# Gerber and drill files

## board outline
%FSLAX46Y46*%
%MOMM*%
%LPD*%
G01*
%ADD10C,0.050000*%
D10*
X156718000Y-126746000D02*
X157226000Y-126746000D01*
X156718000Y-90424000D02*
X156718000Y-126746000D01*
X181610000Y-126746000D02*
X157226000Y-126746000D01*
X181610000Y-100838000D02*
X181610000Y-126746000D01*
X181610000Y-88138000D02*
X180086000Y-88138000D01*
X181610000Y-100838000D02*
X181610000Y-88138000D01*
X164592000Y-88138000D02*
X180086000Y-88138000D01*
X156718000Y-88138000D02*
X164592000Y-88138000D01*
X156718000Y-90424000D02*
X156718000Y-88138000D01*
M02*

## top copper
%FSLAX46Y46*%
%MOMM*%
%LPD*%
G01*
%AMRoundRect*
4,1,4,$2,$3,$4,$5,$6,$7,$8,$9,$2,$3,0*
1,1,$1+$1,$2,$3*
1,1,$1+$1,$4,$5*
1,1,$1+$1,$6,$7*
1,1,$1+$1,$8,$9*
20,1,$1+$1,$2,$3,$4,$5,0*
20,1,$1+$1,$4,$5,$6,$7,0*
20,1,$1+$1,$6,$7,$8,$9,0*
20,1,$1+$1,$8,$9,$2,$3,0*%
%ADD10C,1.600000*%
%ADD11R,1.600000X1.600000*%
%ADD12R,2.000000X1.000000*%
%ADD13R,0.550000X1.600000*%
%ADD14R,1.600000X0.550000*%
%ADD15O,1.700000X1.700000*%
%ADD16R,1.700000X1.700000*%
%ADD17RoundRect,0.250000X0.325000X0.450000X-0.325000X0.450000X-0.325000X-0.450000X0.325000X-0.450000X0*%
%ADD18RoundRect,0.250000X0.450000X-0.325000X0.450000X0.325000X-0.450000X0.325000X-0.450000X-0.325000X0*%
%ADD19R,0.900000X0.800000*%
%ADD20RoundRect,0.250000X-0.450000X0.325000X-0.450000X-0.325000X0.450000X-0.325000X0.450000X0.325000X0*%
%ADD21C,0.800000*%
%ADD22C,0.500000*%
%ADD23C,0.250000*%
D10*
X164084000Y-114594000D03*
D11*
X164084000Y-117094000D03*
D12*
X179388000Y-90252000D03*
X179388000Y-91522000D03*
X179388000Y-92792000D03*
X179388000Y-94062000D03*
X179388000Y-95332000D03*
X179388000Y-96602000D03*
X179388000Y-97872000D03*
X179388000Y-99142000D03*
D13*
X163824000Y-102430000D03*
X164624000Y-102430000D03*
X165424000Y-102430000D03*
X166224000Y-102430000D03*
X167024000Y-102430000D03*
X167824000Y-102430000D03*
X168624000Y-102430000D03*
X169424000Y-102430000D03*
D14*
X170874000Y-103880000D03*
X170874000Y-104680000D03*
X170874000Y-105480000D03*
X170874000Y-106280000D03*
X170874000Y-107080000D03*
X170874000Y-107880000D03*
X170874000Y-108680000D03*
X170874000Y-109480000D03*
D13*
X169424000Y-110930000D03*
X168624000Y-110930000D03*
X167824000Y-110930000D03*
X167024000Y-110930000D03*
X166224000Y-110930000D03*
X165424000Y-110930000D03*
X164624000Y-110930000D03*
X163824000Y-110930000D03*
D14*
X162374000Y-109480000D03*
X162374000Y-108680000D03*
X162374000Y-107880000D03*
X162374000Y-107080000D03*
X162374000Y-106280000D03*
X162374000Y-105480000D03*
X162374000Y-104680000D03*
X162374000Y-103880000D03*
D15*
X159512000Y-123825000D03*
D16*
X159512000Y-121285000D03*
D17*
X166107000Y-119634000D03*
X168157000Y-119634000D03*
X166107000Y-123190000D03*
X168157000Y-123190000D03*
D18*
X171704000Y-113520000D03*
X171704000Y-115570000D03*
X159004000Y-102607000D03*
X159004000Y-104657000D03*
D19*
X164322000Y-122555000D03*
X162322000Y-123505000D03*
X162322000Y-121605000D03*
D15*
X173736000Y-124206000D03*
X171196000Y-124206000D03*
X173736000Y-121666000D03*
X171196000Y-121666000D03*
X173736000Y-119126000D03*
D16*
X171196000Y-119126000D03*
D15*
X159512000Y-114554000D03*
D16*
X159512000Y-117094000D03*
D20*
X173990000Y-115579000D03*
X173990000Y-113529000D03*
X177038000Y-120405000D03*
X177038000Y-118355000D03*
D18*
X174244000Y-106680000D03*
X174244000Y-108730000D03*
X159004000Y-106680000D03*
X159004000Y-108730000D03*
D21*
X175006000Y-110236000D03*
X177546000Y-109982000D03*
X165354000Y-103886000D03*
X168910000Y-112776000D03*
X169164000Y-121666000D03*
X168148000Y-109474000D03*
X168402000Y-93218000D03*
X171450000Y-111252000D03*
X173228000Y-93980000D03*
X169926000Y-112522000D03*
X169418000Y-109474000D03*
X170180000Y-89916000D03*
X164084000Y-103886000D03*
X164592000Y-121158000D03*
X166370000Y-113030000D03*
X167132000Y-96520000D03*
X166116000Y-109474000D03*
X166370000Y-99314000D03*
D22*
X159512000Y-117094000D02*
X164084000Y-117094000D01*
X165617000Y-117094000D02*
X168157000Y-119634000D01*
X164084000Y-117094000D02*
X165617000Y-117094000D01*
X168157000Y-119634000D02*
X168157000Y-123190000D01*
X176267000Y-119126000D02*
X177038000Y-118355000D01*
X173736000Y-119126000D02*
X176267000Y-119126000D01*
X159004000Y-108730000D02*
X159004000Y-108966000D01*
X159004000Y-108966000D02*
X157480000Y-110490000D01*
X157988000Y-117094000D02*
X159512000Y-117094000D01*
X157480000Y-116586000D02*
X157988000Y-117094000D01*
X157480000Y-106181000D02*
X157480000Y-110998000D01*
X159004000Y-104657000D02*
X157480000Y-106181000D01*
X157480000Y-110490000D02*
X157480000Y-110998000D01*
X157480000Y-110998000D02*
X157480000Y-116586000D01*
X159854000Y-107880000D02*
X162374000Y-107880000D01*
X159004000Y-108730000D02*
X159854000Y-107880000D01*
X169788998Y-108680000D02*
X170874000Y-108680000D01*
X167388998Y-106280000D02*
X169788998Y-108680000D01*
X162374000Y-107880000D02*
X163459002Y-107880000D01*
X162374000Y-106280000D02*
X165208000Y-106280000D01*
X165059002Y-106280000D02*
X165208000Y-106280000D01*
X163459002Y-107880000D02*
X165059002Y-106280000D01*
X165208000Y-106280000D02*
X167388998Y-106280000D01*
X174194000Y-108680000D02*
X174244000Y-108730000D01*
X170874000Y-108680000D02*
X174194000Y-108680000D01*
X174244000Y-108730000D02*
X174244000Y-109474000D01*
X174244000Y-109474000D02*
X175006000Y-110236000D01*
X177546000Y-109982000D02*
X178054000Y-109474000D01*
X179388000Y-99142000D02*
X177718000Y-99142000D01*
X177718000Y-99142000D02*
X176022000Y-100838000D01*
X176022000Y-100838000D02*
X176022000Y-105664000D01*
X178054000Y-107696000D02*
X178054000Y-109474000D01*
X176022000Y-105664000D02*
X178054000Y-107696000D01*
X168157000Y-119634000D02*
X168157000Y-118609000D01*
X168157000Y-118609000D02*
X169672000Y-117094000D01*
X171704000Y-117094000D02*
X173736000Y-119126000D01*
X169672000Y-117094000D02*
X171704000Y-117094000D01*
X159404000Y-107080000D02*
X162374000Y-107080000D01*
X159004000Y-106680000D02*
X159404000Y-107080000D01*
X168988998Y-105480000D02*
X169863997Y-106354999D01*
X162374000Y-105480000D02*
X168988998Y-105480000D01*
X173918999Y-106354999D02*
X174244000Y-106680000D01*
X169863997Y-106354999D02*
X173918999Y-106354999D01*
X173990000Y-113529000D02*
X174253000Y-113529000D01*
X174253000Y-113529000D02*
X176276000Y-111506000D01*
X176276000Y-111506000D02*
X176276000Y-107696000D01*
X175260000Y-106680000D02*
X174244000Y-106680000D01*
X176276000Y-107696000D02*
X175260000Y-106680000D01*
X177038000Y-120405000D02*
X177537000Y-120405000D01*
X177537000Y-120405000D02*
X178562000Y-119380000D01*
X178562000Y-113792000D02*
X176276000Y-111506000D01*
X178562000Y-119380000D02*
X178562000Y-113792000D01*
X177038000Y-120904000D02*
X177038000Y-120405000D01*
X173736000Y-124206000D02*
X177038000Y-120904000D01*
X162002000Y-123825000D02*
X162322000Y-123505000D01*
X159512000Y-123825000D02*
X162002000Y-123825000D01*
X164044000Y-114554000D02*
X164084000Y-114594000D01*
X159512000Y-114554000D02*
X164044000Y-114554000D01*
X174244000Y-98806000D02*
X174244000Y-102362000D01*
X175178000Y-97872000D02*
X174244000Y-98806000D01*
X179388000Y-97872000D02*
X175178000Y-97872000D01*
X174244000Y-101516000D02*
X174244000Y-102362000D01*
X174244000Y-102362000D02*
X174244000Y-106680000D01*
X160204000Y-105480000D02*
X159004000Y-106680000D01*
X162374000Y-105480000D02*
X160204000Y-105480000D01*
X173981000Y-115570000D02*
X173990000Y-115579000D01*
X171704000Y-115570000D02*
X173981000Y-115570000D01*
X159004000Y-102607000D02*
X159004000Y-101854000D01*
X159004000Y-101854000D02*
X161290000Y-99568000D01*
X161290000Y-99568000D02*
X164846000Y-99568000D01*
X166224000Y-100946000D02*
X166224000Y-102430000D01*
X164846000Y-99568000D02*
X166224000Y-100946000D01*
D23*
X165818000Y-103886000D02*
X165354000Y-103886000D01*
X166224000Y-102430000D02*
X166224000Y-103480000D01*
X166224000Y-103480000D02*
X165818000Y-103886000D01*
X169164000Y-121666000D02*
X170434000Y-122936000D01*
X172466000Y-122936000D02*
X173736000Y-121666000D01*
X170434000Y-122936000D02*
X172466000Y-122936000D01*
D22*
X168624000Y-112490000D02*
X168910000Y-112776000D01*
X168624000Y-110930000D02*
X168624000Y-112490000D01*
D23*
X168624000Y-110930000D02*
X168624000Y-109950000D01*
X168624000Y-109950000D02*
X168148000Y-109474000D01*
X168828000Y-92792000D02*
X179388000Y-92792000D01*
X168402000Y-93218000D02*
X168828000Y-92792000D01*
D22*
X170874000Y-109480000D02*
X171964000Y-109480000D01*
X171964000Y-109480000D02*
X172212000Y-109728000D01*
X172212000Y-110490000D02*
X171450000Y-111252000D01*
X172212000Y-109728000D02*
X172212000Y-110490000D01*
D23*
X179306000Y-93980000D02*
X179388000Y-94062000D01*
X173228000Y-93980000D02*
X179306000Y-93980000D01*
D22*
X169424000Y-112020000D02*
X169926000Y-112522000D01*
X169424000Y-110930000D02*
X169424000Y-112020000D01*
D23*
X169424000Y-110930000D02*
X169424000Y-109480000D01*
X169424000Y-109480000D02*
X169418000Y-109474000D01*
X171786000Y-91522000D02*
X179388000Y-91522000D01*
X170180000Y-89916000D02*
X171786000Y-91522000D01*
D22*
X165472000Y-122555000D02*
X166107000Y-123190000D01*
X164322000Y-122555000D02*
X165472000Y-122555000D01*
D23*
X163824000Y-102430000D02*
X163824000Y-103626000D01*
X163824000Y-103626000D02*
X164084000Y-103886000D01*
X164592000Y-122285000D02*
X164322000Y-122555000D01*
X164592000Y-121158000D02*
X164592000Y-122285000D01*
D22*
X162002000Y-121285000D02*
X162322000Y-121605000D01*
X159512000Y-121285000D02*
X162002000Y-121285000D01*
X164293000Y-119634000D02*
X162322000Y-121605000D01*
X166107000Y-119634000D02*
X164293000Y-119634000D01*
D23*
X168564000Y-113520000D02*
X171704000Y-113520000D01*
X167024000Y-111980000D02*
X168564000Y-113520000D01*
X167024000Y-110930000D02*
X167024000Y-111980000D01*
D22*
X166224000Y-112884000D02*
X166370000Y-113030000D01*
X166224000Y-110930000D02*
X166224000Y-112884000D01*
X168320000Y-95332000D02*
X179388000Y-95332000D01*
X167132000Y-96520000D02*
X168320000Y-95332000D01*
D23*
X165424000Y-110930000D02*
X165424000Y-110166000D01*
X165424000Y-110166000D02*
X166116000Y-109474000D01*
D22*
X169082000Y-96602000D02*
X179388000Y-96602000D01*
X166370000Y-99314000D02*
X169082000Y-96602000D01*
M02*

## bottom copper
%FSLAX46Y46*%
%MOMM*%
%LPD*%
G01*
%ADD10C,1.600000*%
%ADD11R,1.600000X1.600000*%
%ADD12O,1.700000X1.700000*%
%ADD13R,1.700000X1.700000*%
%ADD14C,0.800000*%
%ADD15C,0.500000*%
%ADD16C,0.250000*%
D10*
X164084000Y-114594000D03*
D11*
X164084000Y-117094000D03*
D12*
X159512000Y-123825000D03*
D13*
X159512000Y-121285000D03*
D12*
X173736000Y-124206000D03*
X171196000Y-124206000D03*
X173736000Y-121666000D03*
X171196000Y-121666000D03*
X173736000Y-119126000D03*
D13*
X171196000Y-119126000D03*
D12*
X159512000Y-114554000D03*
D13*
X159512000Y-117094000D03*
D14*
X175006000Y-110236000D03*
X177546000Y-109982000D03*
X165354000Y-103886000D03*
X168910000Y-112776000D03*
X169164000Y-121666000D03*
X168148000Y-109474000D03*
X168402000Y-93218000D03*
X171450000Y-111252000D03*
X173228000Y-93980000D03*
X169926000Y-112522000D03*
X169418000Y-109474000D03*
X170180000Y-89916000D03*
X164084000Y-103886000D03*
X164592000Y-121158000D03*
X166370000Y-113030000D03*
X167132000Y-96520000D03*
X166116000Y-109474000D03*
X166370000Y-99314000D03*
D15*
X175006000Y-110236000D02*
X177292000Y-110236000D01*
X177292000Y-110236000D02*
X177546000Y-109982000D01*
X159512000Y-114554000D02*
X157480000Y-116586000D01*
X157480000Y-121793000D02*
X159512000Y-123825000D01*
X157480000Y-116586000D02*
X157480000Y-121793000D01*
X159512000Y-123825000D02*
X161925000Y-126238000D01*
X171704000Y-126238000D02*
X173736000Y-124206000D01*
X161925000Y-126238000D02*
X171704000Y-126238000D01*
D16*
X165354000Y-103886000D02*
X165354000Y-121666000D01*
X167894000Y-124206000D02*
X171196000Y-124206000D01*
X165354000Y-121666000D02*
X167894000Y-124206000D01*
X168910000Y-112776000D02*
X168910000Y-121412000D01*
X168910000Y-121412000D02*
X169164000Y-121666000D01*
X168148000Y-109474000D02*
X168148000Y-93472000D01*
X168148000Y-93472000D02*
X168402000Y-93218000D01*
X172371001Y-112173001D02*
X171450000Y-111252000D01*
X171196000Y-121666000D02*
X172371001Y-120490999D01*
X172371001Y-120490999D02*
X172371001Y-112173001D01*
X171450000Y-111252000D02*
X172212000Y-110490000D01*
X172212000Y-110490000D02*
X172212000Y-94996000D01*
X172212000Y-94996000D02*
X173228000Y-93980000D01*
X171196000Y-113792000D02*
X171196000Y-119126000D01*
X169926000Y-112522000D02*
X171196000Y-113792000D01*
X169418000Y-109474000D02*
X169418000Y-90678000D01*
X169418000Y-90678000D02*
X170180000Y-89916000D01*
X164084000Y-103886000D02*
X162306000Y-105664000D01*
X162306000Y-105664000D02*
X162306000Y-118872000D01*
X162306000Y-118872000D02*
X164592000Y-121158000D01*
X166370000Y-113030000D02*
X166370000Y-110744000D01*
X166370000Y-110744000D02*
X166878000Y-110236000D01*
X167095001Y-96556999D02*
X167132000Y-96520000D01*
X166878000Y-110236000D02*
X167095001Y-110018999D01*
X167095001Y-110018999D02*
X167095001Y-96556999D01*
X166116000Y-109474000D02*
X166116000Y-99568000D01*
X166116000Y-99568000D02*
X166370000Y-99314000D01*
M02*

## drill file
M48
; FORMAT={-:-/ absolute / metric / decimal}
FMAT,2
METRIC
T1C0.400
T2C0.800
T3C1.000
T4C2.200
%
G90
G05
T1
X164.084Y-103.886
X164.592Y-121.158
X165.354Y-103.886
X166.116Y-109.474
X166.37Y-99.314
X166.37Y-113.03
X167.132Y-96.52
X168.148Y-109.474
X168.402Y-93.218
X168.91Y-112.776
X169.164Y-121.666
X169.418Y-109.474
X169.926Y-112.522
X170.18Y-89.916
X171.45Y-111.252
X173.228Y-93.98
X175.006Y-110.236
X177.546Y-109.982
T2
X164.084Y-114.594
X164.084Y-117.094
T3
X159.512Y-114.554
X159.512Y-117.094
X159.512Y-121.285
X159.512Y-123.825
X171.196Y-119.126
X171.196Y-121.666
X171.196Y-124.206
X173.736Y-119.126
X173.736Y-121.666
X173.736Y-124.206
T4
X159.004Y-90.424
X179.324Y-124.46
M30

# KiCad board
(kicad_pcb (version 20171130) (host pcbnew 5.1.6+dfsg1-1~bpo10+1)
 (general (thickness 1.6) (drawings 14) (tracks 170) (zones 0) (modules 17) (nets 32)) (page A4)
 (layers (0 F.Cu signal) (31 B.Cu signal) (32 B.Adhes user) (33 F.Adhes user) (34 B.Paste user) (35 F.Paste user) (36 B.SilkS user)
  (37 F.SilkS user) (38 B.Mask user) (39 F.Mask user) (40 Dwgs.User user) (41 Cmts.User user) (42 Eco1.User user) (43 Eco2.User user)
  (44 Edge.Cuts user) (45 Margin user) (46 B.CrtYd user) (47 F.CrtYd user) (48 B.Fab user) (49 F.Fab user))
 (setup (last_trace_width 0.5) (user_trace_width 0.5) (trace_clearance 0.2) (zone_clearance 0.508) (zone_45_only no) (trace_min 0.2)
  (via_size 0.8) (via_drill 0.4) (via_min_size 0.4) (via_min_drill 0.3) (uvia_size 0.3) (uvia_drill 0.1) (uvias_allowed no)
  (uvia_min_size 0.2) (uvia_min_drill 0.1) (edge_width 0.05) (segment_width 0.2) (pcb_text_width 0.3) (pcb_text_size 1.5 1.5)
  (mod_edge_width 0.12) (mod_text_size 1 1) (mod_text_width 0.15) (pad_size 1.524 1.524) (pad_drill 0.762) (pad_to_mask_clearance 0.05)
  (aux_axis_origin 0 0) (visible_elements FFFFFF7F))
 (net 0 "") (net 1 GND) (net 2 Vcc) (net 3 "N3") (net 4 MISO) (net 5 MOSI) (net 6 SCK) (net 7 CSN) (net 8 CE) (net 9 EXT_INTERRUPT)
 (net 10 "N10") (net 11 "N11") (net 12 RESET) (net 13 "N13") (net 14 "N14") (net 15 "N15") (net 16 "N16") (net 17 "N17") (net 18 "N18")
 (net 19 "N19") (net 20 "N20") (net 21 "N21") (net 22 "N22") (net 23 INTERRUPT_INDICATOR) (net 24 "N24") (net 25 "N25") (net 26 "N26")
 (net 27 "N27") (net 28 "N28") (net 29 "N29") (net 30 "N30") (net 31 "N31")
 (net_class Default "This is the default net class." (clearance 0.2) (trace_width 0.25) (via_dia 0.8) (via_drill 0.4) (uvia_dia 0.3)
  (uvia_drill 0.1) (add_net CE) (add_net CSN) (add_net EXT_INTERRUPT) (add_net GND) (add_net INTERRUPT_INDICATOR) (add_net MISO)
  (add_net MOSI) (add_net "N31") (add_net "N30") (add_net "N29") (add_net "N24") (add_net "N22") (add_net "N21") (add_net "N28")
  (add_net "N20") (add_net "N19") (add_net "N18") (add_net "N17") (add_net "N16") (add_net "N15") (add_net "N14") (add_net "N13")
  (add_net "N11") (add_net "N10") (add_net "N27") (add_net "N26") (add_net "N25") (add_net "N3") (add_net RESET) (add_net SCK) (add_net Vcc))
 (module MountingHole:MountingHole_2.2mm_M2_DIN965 (layer F.Cu) (at 179.324 124.46)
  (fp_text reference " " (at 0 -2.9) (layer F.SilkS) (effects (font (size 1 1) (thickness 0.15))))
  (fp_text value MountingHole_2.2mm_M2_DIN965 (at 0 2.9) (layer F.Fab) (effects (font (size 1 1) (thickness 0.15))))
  (pad 1 np_thru_hole circle (at 0 0) (size 2.2 2.2) (drill 2.2) (layers *.Cu *.Mask)))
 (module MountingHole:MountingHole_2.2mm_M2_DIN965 (layer F.Cu) (at 159.004 90.424)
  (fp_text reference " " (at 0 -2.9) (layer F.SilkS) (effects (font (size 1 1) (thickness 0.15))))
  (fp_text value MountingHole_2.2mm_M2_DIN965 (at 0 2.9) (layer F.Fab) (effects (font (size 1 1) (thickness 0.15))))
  (pad 1 np_thru_hole circle (at 0 0) (size 2.2 2.2) (drill 2.2) (layers *.Cu *.Mask)))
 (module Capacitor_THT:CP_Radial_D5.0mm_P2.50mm (layer F.Cu) (at 164.084 117.094 90)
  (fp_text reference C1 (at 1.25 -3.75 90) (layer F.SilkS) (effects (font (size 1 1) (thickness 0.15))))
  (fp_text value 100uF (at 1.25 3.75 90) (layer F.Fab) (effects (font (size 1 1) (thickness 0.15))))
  (pad 2 thru_hole circle (at 2.5 0 90) (size 1.6 1.6) (drill 0.8) (layers *.Cu *.Mask) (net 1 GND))
  (pad 1 thru_hole rect (at 0 0 90) (size 1.6 1.6) (drill 0.8) (layers *.Cu *.Mask) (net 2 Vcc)))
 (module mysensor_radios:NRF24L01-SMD (layer F.Cu) (at 170.688 94.742 90)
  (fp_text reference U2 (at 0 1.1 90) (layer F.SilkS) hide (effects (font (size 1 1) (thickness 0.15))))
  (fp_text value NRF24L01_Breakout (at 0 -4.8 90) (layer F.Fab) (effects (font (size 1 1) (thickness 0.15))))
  (pad 8 smd rect (at 4.49 8.7 90) (size 1 2) (layers F.Cu F.Paste F.Mask) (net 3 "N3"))
  (pad 7 smd rect (at 3.22 8.7 90) (size 1 2) (layers F.Cu F.Paste F.Mask) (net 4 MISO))
  (pad 6 smd rect (at 1.95 8.7 90) (size 1 2) (layers F.Cu F.Paste F.Mask) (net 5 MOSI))
  (pad 5 smd rect (at 0.68 8.7 90) (size 1 2) (layers F.Cu F.Paste F.Mask) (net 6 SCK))
  (pad 4 smd rect (at -0.59 8.7 90) (size 1 2) (layers F.Cu F.Paste F.Mask) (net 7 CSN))
  (pad 3 smd rect (at -1.86 8.7 90) (size 1 2) (layers F.Cu F.Paste F.Mask) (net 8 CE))
  (pad 1 smd rect (at -3.13 8.7 90) (size 1 2) (layers F.Cu F.Paste F.Mask) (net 1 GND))
  (pad 2 smd rect (at -4.4 8.7 90) (size 1 2) (layers F.Cu F.Paste F.Mask) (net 2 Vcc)))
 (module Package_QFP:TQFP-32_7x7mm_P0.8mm (layer F.Cu) (at 166.624 106.68)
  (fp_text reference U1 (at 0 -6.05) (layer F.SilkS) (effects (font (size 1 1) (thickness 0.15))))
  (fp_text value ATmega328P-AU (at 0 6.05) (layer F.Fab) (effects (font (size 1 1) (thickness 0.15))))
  (pad 32 smd rect (at -2.8 -4.25 90) (size 1.6 0.55) (layers F.Cu F.Paste F.Mask) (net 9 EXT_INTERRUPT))
  (pad 31 smd rect (at -2 -4.25 90) (size 1.6 0.55) (layers F.Cu F.Paste F.Mask) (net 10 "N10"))
  (pad 30 smd rect (at -1.2 -4.25 90) (size 1.6 0.55) (layers F.Cu F.Paste F.Mask) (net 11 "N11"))
  (pad 29 smd rect (at -0.4 -4.25 90) (size 1.6 0.55) (layers F.Cu F.Paste F.Mask) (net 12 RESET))
  (pad 28 smd rect (at 0.4 -4.25 90) (size 1.6 0.55) (layers F.Cu F.Paste F.Mask) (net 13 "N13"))
  (pad 27 smd rect (at 1.2 -4.25 90) (size 1.6 0.55) (layers F.Cu F.Paste F.Mask) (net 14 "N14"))
  (pad 26 smd rect (at 2 -4.25 90) (size 1.6 0.55) (layers F.Cu F.Paste F.Mask) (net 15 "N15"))
  (pad 25 smd rect (at 2.8 -4.25 90) (size 1.6 0.55) (layers F.Cu F.Paste F.Mask) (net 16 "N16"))
  (pad 24 smd rect (at 4.25 -2.8) (size 1.6 0.55) (layers F.Cu F.Paste F.Mask) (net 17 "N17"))
  (pad 23 smd rect (at 4.25 -2) (size 1.6 0.55) (layers F.Cu F.Paste F.Mask) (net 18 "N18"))
  (pad 22 smd rect (at 4.25 -1.2) (size 1.6 0.55) (layers F.Cu F.Paste F.Mask) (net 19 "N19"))
  (pad 21 smd rect (at 4.25 -0.4) (size 1.6 0.55) (layers F.Cu F.Paste F.Mask) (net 1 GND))
  (pad 20 smd rect (at 4.25 0.4) (size 1.6 0.55) (layers F.Cu F.Paste F.Mask) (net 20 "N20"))
  (pad 19 smd rect (at 4.25 1.2) (size 1.6 0.55) (layers F.Cu F.Paste F.Mask) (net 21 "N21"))
  (pad 18 smd rect (at 4.25 2) (size 1.6 0.55) (layers F.Cu F.Paste F.Mask) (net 2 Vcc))
  (pad 17 smd rect (at 4.25 2.8) (size 1.6 0.55) (layers F.Cu F.Paste F.Mask) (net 6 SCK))
  (pad 16 smd rect (at 2.8 4.25 90) (size 1.6 0.55) (layers F.Cu F.Paste F.Mask) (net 4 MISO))
  (pad 15 smd rect (at 2 4.25 90) (size 1.6 0.55) (layers F.Cu F.Paste F.Mask) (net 5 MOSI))
  (pad 14 smd rect (at 1.2 4.25 90) (size 1.6 0.55) (layers F.Cu F.Paste F.Mask) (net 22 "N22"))
  (pad 13 smd rect (at 0.4 4.25 90) (size 1.6 0.55) (layers F.Cu F.Paste F.Mask) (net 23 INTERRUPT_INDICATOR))
  (pad 12 smd rect (at -0.4 4.25 90) (size 1.6 0.55) (layers F.Cu F.Paste F.Mask) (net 7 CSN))
  (pad 11 smd rect (at -1.2 4.25 90) (size 1.6 0.55) (layers F.Cu F.Paste F.Mask) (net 8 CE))
  (pad 10 smd rect (at -2 4.25 90) (size 1.6 0.55) (layers F.Cu F.Paste F.Mask) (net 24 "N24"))
  (pad 9 smd rect (at -2.8 4.25 90) (size 1.6 0.55) (layers F.Cu F.Paste F.Mask) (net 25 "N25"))
  (pad 8 smd rect (at -4.25 2.8) (size 1.6 0.55) (layers F.Cu F.Paste F.Mask) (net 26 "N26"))
  (pad 7 smd rect (at -4.25 2) (size 1.6 0.55) (layers F.Cu F.Paste F.Mask) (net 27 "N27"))
  (pad 6 smd rect (at -4.25 1.2) (size 1.6 0.55) (layers F.Cu F.Paste F.Mask) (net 2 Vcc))
  (pad 5 smd rect (at -4.25 0.4) (size 1.6 0.55) (layers F.Cu F.Paste F.Mask) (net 1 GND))
  (pad 4 smd rect (at -4.25 -0.4) (size 1.6 0.55) (layers F.Cu F.Paste F.Mask) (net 2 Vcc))
  (pad 3 smd rect (at -4.25 -1.2) (size 1.6 0.55) (layers F.Cu F.Paste F.Mask) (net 1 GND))
  (pad 2 smd rect (at -4.25 -2) (size 1.6 0.55) (layers F.Cu F.Paste F.Mask) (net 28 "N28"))
  (pad 1 smd rect (at -4.25 -2.8) (size 1.6 0.55) (layers F.Cu F.Paste F.Mask) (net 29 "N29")))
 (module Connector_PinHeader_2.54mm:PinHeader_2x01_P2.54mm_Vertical (layer F.Cu) (at 159.512 121.285 270)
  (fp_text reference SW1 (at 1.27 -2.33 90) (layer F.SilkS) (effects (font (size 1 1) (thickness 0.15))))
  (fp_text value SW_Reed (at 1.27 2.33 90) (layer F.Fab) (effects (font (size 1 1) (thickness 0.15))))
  (pad 2 thru_hole oval (at 2.54 0 270) (size 1.7 1.7) (drill 1) (layers *.Cu *.Mask) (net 1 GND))
  (pad 1 thru_hole rect (at 0 0 270) (size 1.7 1.7) (drill 1) (layers *.Cu *.Mask) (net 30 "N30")))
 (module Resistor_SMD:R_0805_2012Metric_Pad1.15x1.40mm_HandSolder (layer F.Cu) (at 167.132 119.634 180)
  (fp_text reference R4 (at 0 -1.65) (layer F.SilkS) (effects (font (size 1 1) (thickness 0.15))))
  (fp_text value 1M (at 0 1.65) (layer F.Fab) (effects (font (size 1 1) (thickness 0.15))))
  (pad 2 smd roundrect (at 1.025 0 180) (size 1.15 1.4) (layers F.Cu F.Paste F.Mask) (roundrect_rratio 0.217391) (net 30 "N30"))
  (pad 1 smd roundrect (at -1.025 0 180) (size 1.15 1.4) (layers F.Cu F.Paste F.Mask) (roundrect_rratio 0.217391) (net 2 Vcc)))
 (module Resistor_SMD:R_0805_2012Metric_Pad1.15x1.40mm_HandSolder (layer F.Cu) (at 167.132 123.19 180)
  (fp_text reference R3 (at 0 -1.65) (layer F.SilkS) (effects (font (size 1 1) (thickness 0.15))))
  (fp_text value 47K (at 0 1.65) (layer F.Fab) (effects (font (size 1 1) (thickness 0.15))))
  (pad 2 smd roundrect (at 1.025 0 180) (size 1.15 1.4) (layers F.Cu F.Paste F.Mask) (roundrect_rratio 0.217391) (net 9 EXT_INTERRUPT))
  (pad 1 smd roundrect (at -1.025 0 180) (size 1.15 1.4) (layers F.Cu F.Paste F.Mask) (roundrect_rratio 0.217391) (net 2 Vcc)))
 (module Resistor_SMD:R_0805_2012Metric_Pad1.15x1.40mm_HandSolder (layer F.Cu) (at 171.704 114.545 90)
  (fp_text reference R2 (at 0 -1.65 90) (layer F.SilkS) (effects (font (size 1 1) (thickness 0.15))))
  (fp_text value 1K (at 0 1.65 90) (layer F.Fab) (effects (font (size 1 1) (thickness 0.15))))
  (pad 2 smd roundrect (at 1.025 0 90) (size 1.15 1.4) (layers F.Cu F.Paste F.Mask) (roundrect_rratio 0.217391) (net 23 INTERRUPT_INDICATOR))
  (pad 1 smd roundrect (at -1.025 0 90) (size 1.15 1.4) (layers F.Cu F.Paste F.Mask) (roundrect_rratio 0.217391) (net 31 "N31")))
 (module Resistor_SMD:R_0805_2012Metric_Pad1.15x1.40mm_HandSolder (layer F.Cu) (at 159.004 103.632 90)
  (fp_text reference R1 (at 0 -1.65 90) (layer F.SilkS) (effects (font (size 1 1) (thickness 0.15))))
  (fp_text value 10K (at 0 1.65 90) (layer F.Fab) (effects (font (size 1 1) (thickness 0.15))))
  (pad 2 smd roundrect (at 1.025 0 90) (size 1.15 1.4) (layers F.Cu F.Paste F.Mask) (roundrect_rratio 0.217391) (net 12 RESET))
  (pad 1 smd roundrect (at -1.025 0 90) (size 1.15 1.4) (layers F.Cu F.Paste F.Mask) (roundrect_rratio 0.217391) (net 2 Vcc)))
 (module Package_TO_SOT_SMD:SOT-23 (layer F.Cu) (at 163.322 122.555)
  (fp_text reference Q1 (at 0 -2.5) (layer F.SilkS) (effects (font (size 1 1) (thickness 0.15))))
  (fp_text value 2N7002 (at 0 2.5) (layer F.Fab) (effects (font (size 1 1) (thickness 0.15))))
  (pad 3 smd rect (at 1 0) (size 0.9 0.8) (layers F.Cu F.Paste F.Mask) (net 9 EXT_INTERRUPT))
  (pad 2 smd rect (at -1 0.95) (size 0.9 0.8) (layers F.Cu F.Paste F.Mask) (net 1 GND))
  (pad 1 smd rect (at -1 -0.95) (size 0.9 0.8) (layers F.Cu F.Paste F.Mask) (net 30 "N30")))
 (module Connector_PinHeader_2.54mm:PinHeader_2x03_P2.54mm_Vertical (layer F.Cu) (at 171.196 119.126)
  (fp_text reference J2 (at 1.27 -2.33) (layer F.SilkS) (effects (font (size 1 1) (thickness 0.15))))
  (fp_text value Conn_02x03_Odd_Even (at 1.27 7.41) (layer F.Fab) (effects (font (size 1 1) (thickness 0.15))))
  (pad 6 thru_hole oval (at 2.54 5.08) (size 1.7 1.7) (drill 1) (layers *.Cu *.Mask) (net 1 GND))
  (pad 5 thru_hole oval (at 0 5.08) (size 1.7 1.7) (drill 1) (layers *.Cu *.Mask) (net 12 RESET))
  (pad 4 thru_hole oval (at 2.54 2.54) (size 1.7 1.7) (drill 1) (layers *.Cu *.Mask) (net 5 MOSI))
  (pad 3 thru_hole oval (at 0 2.54) (size 1.7 1.7) (drill 1) (layers *.Cu *.Mask) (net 6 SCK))
  (pad 2 thru_hole oval (at 2.54 0) (size 1.7 1.7) (drill 1) (layers *.Cu *.Mask) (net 2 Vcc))
  (pad 1 thru_hole rect (at 0 0) (size 1.7 1.7) (drill 1) (layers *.Cu *.Mask) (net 4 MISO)))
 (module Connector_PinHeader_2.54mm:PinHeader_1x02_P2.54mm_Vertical (layer F.Cu) (at 159.512 117.094 180)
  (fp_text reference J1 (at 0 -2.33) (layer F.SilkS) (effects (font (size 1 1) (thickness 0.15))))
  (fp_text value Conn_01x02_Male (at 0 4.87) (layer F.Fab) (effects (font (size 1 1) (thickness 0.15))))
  (pad 2 thru_hole oval (at 0 2.54 180) (size 1.7 1.7) (drill 1) (layers *.Cu *.Mask) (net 1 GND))
  (pad 1 thru_hole rect (at 0 0 180) (size 1.7 1.7) (drill 1) (layers *.Cu *.Mask) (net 2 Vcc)))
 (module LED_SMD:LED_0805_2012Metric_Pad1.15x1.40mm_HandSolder (layer F.Cu) (at 173.99 114.554 270)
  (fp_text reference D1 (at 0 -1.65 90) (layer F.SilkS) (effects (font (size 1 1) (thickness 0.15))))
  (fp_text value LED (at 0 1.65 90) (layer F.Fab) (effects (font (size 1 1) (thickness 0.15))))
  (pad 2 smd roundrect (at 1.025 0 270) (size 1.15 1.4) (layers F.Cu F.Paste F.Mask) (roundrect_rratio 0.217391) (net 31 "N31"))
  (pad 1 smd roundrect (at -1.025 0 270) (size 1.15 1.4) (layers F.Cu F.Paste F.Mask) (roundrect_rratio 0.217391) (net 1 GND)))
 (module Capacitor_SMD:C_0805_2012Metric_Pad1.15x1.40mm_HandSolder (layer F.Cu) (at 177.038 119.38 270)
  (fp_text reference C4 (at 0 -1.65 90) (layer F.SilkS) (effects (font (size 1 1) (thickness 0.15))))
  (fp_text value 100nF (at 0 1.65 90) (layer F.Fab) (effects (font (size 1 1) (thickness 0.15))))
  (pad 2 smd roundrect (at 1.025 0 270) (size 1.15 1.4) (layers F.Cu F.Paste F.Mask) (roundrect_rratio 0.217391) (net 1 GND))
  (pad 1 smd roundrect (at -1.025 0 270) (size 1.15 1.4) (layers F.Cu F.Paste F.Mask) (roundrect_rratio 0.217391) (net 2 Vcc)))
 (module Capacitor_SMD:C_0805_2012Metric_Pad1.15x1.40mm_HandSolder (layer F.Cu) (at 174.244 107.705 90)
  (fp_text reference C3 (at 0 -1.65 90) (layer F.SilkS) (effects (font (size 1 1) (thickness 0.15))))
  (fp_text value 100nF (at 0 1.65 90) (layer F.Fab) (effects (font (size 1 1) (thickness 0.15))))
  (pad 2 smd roundrect (at 1.025 0 90) (size 1.15 1.4) (layers F.Cu F.Paste F.Mask) (roundrect_rratio 0.217391) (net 1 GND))
  (pad 1 smd roundrect (at -1.025 0 90) (size 1.15 1.4) (layers F.Cu F.Paste F.Mask) (roundrect_rratio 0.217391) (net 2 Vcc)))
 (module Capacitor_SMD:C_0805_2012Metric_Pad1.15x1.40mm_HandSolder (layer F.Cu) (at 159.004 107.705 90)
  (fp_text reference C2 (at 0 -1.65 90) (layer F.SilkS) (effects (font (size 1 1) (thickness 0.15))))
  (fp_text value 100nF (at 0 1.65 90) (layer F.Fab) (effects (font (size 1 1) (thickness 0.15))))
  (pad 2 smd roundrect (at 1.025 0 90) (size 1.15 1.4) (layers F.Cu F.Paste F.Mask) (roundrect_rratio 0.217391) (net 1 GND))
  (pad 1 smd roundrect (at -1.025 0 90) (size 1.15 1.4) (layers F.Cu F.Paste F.Mask) (roundrect_rratio 0.217391) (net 2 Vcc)))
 (gr_line (start 156.718 126.746) (end 157.226 126.746) (layer Edge.Cuts) (width 0.05))
 (gr_line (start 156.718 90.424) (end 156.718 126.746) (layer Edge.Cuts) (width 0.05))
 (gr_line (start 181.61 126.746) (end 157.226 126.746) (layer Edge.Cuts) (width 0.05))
 (gr_line (start 181.61 100.838) (end 181.61 126.746) (layer Edge.Cuts) (width 0.05))
 (gr_line (start 181.61 88.138) (end 180.086 88.138) (layer Edge.Cuts) (width 0.05))
 (gr_line (start 181.61 100.838) (end 181.61 88.138) (layer Edge.Cuts) (width 0.05))
 (gr_line (start 164.592 88.138) (end 180.086 88.138) (layer Edge.Cuts) (width 0.05))
 (gr_line (start 156.718 88.138) (end 164.592 88.138) (layer Edge.Cuts) (width 0.05))
 (gr_line (start 156.718 90.424) (end 156.718 88.138) (layer Edge.Cuts) (width 0.05))
 (segment (start 159.512 117.094) (end 164.084 117.094) (width 0.5) (layer F.Cu) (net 2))
 (segment (start 165.617 117.094) (end 168.157 119.634) (width 0.5) (layer F.Cu) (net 2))
 (segment (start 164.084 117.094) (end 165.617 117.094) (width 0.5) (layer F.Cu) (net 2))
 (segment (start 168.157 119.634) (end 168.157 123.19) (width 0.5) (layer F.Cu) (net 2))
 (segment (start 176.267 119.126) (end 177.038 118.355) (width 0.5) (layer F.Cu) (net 2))
 (segment (start 173.736 119.126) (end 176.267 119.126) (width 0.5) (layer F.Cu) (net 2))
 (segment (start 159.004 108.73) (end 159.004 108.966) (width 0.5) (layer F.Cu) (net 2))
 (segment (start 159.004 108.966) (end 157.48 110.49) (width 0.5) (layer F.Cu) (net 2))
 (segment (start 157.988 117.094) (end 159.512 117.094) (width 0.5) (layer F.Cu) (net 2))
 (segment (start 157.48 116.586) (end 157.988 117.094) (width 0.5) (layer F.Cu) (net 2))
 (segment (start 157.48 106.181) (end 157.48 110.998) (width 0.5) (layer F.Cu) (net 2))
 (segment (start 159.004 104.657) (end 157.48 106.181) (width 0.5) (layer F.Cu) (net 2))
 (segment (start 157.48 110.49) (end 157.48 110.998) (width 0.5) (layer F.Cu) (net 2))
 (segment (start 157.48 110.998) (end 157.48 116.586) (width 0.5) (layer F.Cu) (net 2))
 (segment (start 159.854 107.88) (end 162.374 107.88) (width 0.5) (layer F.Cu) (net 2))
 (segment (start 159.004 108.73) (end 159.854 107.88) (width 0.5) (layer F.Cu) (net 2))
 (segment (start 169.788998 108.68) (end 170.874 108.68) (width 0.5) (layer F.Cu) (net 2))
 (segment (start 167.388998 106.28) (end 169.788998 108.68) (width 0.5) (layer F.Cu) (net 2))
 (segment (start 162.374 107.88) (end 163.459002 107.88) (width 0.5) (layer F.Cu) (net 2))
 (segment (start 162.374 106.28) (end 165.208 106.28) (width 0.5) (layer F.Cu) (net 2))
 (segment (start 165.059002 106.28) (end 165.208 106.28) (width 0.5) (layer F.Cu) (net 2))
 (segment (start 163.459002 107.88) (end 165.059002 106.28) (width 0.5) (layer F.Cu) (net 2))
 (segment (start 165.208 106.28) (end 167.388998 106.28) (width 0.5) (layer F.Cu) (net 2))
 (segment (start 174.194 108.68) (end 174.244 108.73) (width 0.5) (layer F.Cu) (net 2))
 (segment (start 170.874 108.68) (end 174.194 108.68) (width 0.5) (layer F.Cu) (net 2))
 (segment (start 174.244 108.73) (end 174.244 109.474) (width 0.5) (layer F.Cu) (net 2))
 (via (at 175.006 110.236) (size 0.8) (drill 0.4) (layers F.Cu B.Cu) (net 2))
 (segment (start 174.244 109.474) (end 175.006 110.236) (width 0.5) (layer F.Cu) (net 2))
 (via (at 177.546 109.982) (size 0.8) (drill 0.4) (layers F.Cu B.Cu) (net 2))
 (segment (start 175.006 110.236) (end 177.292 110.236) (width 0.5) (layer B.Cu) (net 2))
 (segment (start 177.292 110.236) (end 177.546 109.982) (width 0.5) (layer B.Cu) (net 2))
 (segment (start 177.546 109.982) (end 178.054 109.474) (width 0.5) (layer F.Cu) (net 2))
 (segment (start 179.388 99.142) (end 177.718 99.142) (width 0.5) (layer F.Cu) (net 2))
 (segment (start 177.718 99.142) (end 176.022 100.838) (width 0.5) (layer F.Cu) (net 2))
 (segment (start 176.022 100.838) (end 176.022 105.664) (width 0.5) (layer F.Cu) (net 2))
 (segment (start 178.054 107.696) (end 178.054 109.474) (width 0.5) (layer F.Cu) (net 2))
 (segment (start 176.022 105.664) (end 178.054 107.696) (width 0.5) (layer F.Cu) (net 2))
 (segment (start 168.157 119.634) (end 168.157 118.609) (width 0.5) (layer F.Cu) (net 2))
 (segment (start 168.157 118.609) (end 169.672 117.094) (width 0.5) (layer F.Cu) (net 2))
 (segment (start 171.704 117.094) (end 173.736 119.126) (width 0.5) (layer F.Cu) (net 2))
 (segment (start 169.672 117.094) (end 171.704 117.094) (width 0.5) (layer F.Cu) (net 2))
 (segment (start 159.404 107.08) (end 162.374 107.08) (width 0.5) (layer F.Cu) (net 1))
 (segment (start 159.004 106.68) (end 159.404 107.08) (width 0.5) (layer F.Cu) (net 1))
 (segment (start 168.988998 105.48) (end 169.863997 106.354999) (width 0.5) (layer F.Cu) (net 1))
 (segment (start 162.374 105.48) (end 168.988998 105.48) (width 0.5) (layer F.Cu) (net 1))
 (segment (start 173.918999 106.354999) (end 174.244 106.68) (width 0.5) (layer F.Cu) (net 1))
 (segment (start 169.863997 106.354999) (end 173.918999 106.354999) (width 0.5) (layer F.Cu) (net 1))
 (segment (start 173.99 113.529) (end 174.253 113.529) (width 0.5) (layer F.Cu) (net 1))
 (segment (start 174.253 113.529) (end 176.276 111.506) (width 0.5) (layer F.Cu) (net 1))
 (segment (start 176.276 111.506) (end 176.276 107.696) (width 0.5) (layer F.Cu) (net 1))
 (segment (start 175.26 106.68) (end 174.244 106.68) (width 0.5) (layer F.Cu) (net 1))
 (segment (start 176.276 107.696) (end 175.26 106.68) (width 0.5) (layer F.Cu) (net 1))
 (segment (start 177.038 120.405) (end 177.537 120.405) (width 0.5) (layer F.Cu) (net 1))
 (segment (start 177.537 120.405) (end 178.562 119.38) (width 0.5) (layer F.Cu) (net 1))
 (segment (start 178.562 113.792) (end 176.276 111.506) (width 0.5) (layer F.Cu) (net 1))
 (segment (start 178.562 119.38) (end 178.562 113.792) (width 0.5) (layer F.Cu) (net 1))
 (segment (start 177.038 120.904) (end 177.038 120.405) (width 0.5) (layer F.Cu) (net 1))
 (segment (start 173.736 124.206) (end 177.038 120.904) (width 0.5) (layer F.Cu) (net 1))
 (segment (start 162.002 123.825) (end 162.322 123.505) (width 0.5) (layer F.Cu) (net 1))
 (segment (start 159.512 123.825) (end 162.002 123.825) (width 0.5) (layer F.Cu) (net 1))
 (segment (start 164.044 114.554) (end 164.084 114.594) (width 0.5) (layer F.Cu) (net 1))
 (segment (start 159.512 114.554) (end 164.044 114.554) (width 0.5) (layer F.Cu) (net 1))
 (segment (start 159.512 114.554) (end 157.48 116.586) (width 0.5) (layer B.Cu) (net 1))
 (segment (start 157.48 121.793) (end 159.512 123.825) (width 0.5) (layer B.Cu) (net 1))
 (segment (start 157.48 116.586) (end 157.48 121.793) (width 0.5) (layer B.Cu) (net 1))
 (segment (start 159.512 123.825) (end 161.925 126.238) (width 0.5) (layer B.Cu) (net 1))
 (segment (start 171.704 126.238) (end 173.736 124.206) (width 0.5) (layer B.Cu) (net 1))
 (segment (start 161.925 126.238) (end 171.704 126.238) (width 0.5) (layer B.Cu) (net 1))
 (segment (start 174.244 98.806) (end 174.244 102.362) (width 0.5) (layer F.Cu) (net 1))
 (segment (start 175.178 97.872) (end 174.244 98.806) (width 0.5) (layer F.Cu) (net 1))
 (segment (start 179.388 97.872) (end 175.178 97.872) (width 0.5) (layer F.Cu) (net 1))
 (segment (start 174.244 101.516) (end 174.244 102.362) (width 0.5) (layer F.Cu) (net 1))
 (segment (start 174.244 102.362) (end 174.244 106.68) (width 0.5) (layer F.Cu) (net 1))
 (segment (start 160.204 105.48) (end 159.004 106.68) (width 0.5) (layer F.Cu) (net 1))
 (segment (start 162.374 105.48) (end 160.204 105.48) (width 0.5) (layer F.Cu) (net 1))
 (segment (start 173.981 115.57) (end 173.99 115.579) (width 0.5) (layer F.Cu) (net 31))
 (segment (start 171.704 115.57) (end 173.981 115.57) (width 0.5) (layer F.Cu) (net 31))
 (segment (start 159.004 102.607) (end 159.004 101.854) (width 0.5) (layer F.Cu) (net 12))
 (segment (start 159.004 101.854) (end 161.29 99.568) (width 0.5) (layer F.Cu) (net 12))
 (segment (start 161.29 99.568) (end 164.846 99.568) (width 0.5) (layer F.Cu) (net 12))
 (segment (start 166.224 100.946) (end 166.224 102.43) (width 0.5) (layer F.Cu) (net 12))
 (segment (start 164.846 99.568) (end 166.224 100.946) (width 0.5) (layer F.Cu) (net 12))
 (segment (start 165.818 103.886) (end 165.354 103.886) (width 0.25) (layer F.Cu) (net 12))
 (via (at 165.354 103.886) (size 0.8) (drill 0.4) (layers F.Cu B.Cu) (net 12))
 (segment (start 166.224 102.43) (end 166.224 103.48) (width 0.25) (layer F.Cu) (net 12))
 (segment (start 166.224 103.48) (end 165.818 103.886) (width 0.25) (layer F.Cu) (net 12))
 (segment (start 165.354 103.886) (end 165.354 121.666) (width 0.25) (layer B.Cu) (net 12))
 (segment (start 167.894 124.206) (end 171.196 124.206) (width 0.25) (layer B.Cu) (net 12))
 (segment (start 165.354 121.666) (end 167.894 124.206) (width 0.25) (layer B.Cu) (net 12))
 (via (at 168.91 112.776) (size 0.8) (drill 0.4) (layers F.Cu B.Cu) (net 5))
 (via (at 169.164 121.666) (size 0.8) (drill 0.4) (layers F.Cu B.Cu) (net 5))
 (segment (start 168.91 112.776) (end 168.91 121.412) (width 0.25) (layer B.Cu) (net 5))
 (segment (start 168.91 121.412) (end 169.164 121.666) (width 0.25) (layer B.Cu) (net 5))
 (segment (start 169.164 121.666) (end 170.434 122.936) (width 0.25) (layer F.Cu) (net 5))
 (segment (start 172.466 122.936) (end 173.736 121.666) (width 0.25) (layer F.Cu) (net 5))
 (segment (start 170.434 122.936) (end 172.466 122.936) (width 0.25) (layer F.Cu) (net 5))
 (segment (start 168.624 112.49) (end 168.91 112.776) (width 0.5) (layer F.Cu) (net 5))
 (segment (start 168.624 110.93) (end 168.624 112.49) (width 0.5) (layer F.Cu) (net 5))
 (segment (start 168.624 110.93) (end 168.624 109.95) (width 0.25) (layer F.Cu) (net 5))
 (via (at 168.148 109.474) (size 0.8) (drill 0.4) (layers F.Cu B.Cu) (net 5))
 (segment (start 168.624 109.95) (end 168.148 109.474) (width 0.25) (layer F.Cu) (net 5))
 (via (at 168.402 93.218) (size 0.8) (drill 0.4) (layers F.Cu B.Cu) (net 5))
 (segment (start 168.148 109.474) (end 168.148 93.472) (width 0.25) (layer B.Cu) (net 5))
 (segment (start 168.148 93.472) (end 168.402 93.218) (width 0.25) (layer B.Cu) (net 5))
 (segment (start 168.828 92.792) (end 179.388 92.792) (width 0.25) (layer F.Cu) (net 5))
 (segment (start 168.402 93.218) (end 168.828 92.792) (width 0.25) (layer F.Cu) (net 5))
 (via (at 171.45 111.252) (size 0.8) (drill 0.4) (layers F.Cu B.Cu) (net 6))
 (segment (start 172.371001 112.173001) (end 171.45 111.252) (width 0.25) (layer B.Cu) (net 6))
 (segment (start 171.196 121.666) (end 172.371001 120.490999) (width 0.25) (layer B.Cu) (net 6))
 (segment (start 172.371001 120.490999) (end 172.371001 112.173001) (width 0.25) (layer B.Cu) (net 6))
 (segment (start 170.874 109.48) (end 171.964 109.48) (width 0.5) (layer F.Cu) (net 6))
 (segment (start 171.964 109.48) (end 172.212 109.728) (width 0.5) (layer F.Cu) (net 6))
 (segment (start 172.212 110.49) (end 171.45 111.252) (width 0.5) (layer F.Cu) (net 6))
 (segment (start 172.212 109.728) (end 172.212 110.49) (width 0.5) (layer F.Cu) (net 6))
 (segment (start 171.45 111.252) (end 172.212 110.49) (width 0.25) (layer B.Cu) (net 6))
 (via (at 173.228 93.98) (size 0.8) (drill 0.4) (layers F.Cu B.Cu) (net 6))
 (segment (start 172.212 110.49) (end 172.212 94.996) (width 0.25) (layer B.Cu) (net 6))
 (segment (start 172.212 94.996) (end 173.228 93.98) (width 0.25) (layer B.Cu) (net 6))
 (segment (start 179.306 93.98) (end 179.388 94.062) (width 0.25) (layer F.Cu) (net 6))
 (segment (start 173.228 93.98) (end 179.306 93.98) (width 0.25) (layer F.Cu) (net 6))
 (via (at 169.926 112.522) (size 0.8) (drill 0.4) (layers F.Cu B.Cu) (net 4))
 (segment (start 171.196 113.792) (end 171.196 119.126) (width 0.25) (layer B.Cu) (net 4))
 (segment (start 169.926 112.522) (end 171.196 113.792) (width 0.25) (layer B.Cu) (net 4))
 (segment (start 169.424 112.02) (end 169.926 112.522) (width 0.5) (layer F.Cu) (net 4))
 (segment (start 169.424 110.93) (end 169.424 112.02) (width 0.5) (layer F.Cu) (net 4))
 (via (at 169.418 109.474) (size 0.8) (drill 0.4) (layers F.Cu B.Cu) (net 4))
 (segment (start 169.424 110.93) (end 169.424 109.48) (width 0.25) (layer F.Cu) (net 4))
 (segment (start 169.424 109.48) (end 169.418 109.474) (width 0.25) (layer F.Cu) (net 4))
 (segment (start 169.418 109.474) (end 169.418 90.678) (width 0.25) (layer B.Cu) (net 4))
 (via (at 170.18 89.916) (size 0.8) (drill 0.4) (layers F.Cu B.Cu) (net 4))
 (segment (start 169.418 90.678) (end 170.18 89.916) (width 0.25) (layer B.Cu) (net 4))
 (segment (start 171.786 91.522) (end 179.388 91.522) (width 0.25) (layer F.Cu) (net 4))
 (segment (start 170.18 89.916) (end 171.786 91.522) (width 0.25) (layer F.Cu) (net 4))
 (segment (start 165.472 122.555) (end 166.107 123.19) (width 0.5) (layer F.Cu) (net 9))
 (segment (start 164.322 122.555) (end 165.472 122.555) (width 0.5) (layer F.Cu) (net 9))
 (via (at 164.084 103.886) (size 0.8) (drill 0.4) (layers F.Cu B.Cu) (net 9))
 (segment (start 163.824 102.43) (end 163.824 103.626) (width 0.25) (layer F.Cu) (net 9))
 (segment (start 163.824 103.626) (end 164.084 103.886) (width 0.25) (layer F.Cu) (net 9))
 (segment (start 164.084 103.886) (end 162.306 105.664) (width 0.25) (layer B.Cu) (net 9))
 (via (at 164.592 121.158) (size 0.8) (drill 0.4) (layers F.Cu B.Cu) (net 9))
 (segment (start 162.306 105.664) (end 162.306 118.872) (width 0.25) (layer B.Cu) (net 9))
 (segment (start 162.306 118.872) (end 164.592 121.158) (width 0.25) (layer B.Cu) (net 9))
 (segment (start 164.592 122.285) (end 164.322 122.555) (width 0.25) (layer F.Cu) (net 9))
 (segment (start 164.592 121.158) (end 164.592 122.285) (width 0.25) (layer F.Cu) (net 9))
 (segment (start 162.002 121.285) (end 162.322 121.605) (width 0.5) (layer F.Cu) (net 30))
 (segment (start 159.512 121.285) (end 162.002 121.285) (width 0.5) (layer F.Cu) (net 30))
 (segment (start 164.293 119.634) (end 162.322 121.605) (width 0.5) (layer F.Cu) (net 30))
 (segment (start 166.107 119.634) (end 164.293 119.634) (width 0.5) (layer F.Cu) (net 30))
 (segment (start 168.564 113.52) (end 171.704 113.52) (width 0.25) (layer F.Cu) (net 23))
 (segment (start 167.024 111.98) (end 168.564 113.52) (width 0.25) (layer F.Cu) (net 23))
 (segment (start 167.024 110.93) (end 167.024 111.98) (width 0.25) (layer F.Cu) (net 23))
 (via (at 166.37 113.03) (size 0.8) (drill 0.4) (layers F.Cu B.Cu) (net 7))
 (segment (start 166.37 113.03) (end 166.37 110.744) (width 0.25) (layer B.Cu) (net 7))
 (segment (start 166.37 110.744) (end 166.878 110.236) (width 0.25) (layer B.Cu) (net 7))
 (via (at 167.132 96.52) (size 0.8) (drill 0.4) (layers F.Cu B.Cu) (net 7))
 (segment (start 167.095001 96.556999) (end 167.132 96.52) (width 0.25) (layer B.Cu) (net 7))
 (segment (start 166.878 110.236) (end 167.095001 110.018999) (width 0.25) (layer B.Cu) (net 7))
 (segment (start 167.095001 110.018999) (end 167.095001 96.556999) (width 0.25) (layer B.Cu) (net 7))
 (segment (start 166.224 112.884) (end 166.37 113.03) (width 0.5) (layer F.Cu) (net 7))
 (segment (start 166.224 110.93) (end 166.224 112.884) (width 0.5) (layer F.Cu) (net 7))
 (segment (start 168.32 95.332) (end 179.388 95.332) (width 0.5) (layer F.Cu) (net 7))
 (segment (start 167.132 96.52) (end 168.32 95.332) (width 0.5) (layer F.Cu) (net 7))
 (via (at 166.116 109.474) (size 0.8) (drill 0.4) (layers F.Cu B.Cu) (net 8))
 (segment (start 165.424 110.93) (end 165.424 110.166) (width 0.25) (layer F.Cu) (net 8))
 (segment (start 165.424 110.166) (end 166.116 109.474) (width 0.25) (layer F.Cu) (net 8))
 (via (at 166.37 99.314) (size 0.8) (drill 0.4) (layers F.Cu B.Cu) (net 8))
 (segment (start 166.116 109.474) (end 166.116 99.568) (width 0.25) (layer B.Cu) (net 8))
 (segment (start 166.116 99.568) (end 166.37 99.314) (width 0.25) (layer B.Cu) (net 8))
 (segment (start 169.082 96.602) (end 179.388 96.602) (width 0.5) (layer F.Cu) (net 8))
 (segment (start 166.37 99.314) (end 169.082 96.602) (width 0.5) (layer F.Cu) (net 8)))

